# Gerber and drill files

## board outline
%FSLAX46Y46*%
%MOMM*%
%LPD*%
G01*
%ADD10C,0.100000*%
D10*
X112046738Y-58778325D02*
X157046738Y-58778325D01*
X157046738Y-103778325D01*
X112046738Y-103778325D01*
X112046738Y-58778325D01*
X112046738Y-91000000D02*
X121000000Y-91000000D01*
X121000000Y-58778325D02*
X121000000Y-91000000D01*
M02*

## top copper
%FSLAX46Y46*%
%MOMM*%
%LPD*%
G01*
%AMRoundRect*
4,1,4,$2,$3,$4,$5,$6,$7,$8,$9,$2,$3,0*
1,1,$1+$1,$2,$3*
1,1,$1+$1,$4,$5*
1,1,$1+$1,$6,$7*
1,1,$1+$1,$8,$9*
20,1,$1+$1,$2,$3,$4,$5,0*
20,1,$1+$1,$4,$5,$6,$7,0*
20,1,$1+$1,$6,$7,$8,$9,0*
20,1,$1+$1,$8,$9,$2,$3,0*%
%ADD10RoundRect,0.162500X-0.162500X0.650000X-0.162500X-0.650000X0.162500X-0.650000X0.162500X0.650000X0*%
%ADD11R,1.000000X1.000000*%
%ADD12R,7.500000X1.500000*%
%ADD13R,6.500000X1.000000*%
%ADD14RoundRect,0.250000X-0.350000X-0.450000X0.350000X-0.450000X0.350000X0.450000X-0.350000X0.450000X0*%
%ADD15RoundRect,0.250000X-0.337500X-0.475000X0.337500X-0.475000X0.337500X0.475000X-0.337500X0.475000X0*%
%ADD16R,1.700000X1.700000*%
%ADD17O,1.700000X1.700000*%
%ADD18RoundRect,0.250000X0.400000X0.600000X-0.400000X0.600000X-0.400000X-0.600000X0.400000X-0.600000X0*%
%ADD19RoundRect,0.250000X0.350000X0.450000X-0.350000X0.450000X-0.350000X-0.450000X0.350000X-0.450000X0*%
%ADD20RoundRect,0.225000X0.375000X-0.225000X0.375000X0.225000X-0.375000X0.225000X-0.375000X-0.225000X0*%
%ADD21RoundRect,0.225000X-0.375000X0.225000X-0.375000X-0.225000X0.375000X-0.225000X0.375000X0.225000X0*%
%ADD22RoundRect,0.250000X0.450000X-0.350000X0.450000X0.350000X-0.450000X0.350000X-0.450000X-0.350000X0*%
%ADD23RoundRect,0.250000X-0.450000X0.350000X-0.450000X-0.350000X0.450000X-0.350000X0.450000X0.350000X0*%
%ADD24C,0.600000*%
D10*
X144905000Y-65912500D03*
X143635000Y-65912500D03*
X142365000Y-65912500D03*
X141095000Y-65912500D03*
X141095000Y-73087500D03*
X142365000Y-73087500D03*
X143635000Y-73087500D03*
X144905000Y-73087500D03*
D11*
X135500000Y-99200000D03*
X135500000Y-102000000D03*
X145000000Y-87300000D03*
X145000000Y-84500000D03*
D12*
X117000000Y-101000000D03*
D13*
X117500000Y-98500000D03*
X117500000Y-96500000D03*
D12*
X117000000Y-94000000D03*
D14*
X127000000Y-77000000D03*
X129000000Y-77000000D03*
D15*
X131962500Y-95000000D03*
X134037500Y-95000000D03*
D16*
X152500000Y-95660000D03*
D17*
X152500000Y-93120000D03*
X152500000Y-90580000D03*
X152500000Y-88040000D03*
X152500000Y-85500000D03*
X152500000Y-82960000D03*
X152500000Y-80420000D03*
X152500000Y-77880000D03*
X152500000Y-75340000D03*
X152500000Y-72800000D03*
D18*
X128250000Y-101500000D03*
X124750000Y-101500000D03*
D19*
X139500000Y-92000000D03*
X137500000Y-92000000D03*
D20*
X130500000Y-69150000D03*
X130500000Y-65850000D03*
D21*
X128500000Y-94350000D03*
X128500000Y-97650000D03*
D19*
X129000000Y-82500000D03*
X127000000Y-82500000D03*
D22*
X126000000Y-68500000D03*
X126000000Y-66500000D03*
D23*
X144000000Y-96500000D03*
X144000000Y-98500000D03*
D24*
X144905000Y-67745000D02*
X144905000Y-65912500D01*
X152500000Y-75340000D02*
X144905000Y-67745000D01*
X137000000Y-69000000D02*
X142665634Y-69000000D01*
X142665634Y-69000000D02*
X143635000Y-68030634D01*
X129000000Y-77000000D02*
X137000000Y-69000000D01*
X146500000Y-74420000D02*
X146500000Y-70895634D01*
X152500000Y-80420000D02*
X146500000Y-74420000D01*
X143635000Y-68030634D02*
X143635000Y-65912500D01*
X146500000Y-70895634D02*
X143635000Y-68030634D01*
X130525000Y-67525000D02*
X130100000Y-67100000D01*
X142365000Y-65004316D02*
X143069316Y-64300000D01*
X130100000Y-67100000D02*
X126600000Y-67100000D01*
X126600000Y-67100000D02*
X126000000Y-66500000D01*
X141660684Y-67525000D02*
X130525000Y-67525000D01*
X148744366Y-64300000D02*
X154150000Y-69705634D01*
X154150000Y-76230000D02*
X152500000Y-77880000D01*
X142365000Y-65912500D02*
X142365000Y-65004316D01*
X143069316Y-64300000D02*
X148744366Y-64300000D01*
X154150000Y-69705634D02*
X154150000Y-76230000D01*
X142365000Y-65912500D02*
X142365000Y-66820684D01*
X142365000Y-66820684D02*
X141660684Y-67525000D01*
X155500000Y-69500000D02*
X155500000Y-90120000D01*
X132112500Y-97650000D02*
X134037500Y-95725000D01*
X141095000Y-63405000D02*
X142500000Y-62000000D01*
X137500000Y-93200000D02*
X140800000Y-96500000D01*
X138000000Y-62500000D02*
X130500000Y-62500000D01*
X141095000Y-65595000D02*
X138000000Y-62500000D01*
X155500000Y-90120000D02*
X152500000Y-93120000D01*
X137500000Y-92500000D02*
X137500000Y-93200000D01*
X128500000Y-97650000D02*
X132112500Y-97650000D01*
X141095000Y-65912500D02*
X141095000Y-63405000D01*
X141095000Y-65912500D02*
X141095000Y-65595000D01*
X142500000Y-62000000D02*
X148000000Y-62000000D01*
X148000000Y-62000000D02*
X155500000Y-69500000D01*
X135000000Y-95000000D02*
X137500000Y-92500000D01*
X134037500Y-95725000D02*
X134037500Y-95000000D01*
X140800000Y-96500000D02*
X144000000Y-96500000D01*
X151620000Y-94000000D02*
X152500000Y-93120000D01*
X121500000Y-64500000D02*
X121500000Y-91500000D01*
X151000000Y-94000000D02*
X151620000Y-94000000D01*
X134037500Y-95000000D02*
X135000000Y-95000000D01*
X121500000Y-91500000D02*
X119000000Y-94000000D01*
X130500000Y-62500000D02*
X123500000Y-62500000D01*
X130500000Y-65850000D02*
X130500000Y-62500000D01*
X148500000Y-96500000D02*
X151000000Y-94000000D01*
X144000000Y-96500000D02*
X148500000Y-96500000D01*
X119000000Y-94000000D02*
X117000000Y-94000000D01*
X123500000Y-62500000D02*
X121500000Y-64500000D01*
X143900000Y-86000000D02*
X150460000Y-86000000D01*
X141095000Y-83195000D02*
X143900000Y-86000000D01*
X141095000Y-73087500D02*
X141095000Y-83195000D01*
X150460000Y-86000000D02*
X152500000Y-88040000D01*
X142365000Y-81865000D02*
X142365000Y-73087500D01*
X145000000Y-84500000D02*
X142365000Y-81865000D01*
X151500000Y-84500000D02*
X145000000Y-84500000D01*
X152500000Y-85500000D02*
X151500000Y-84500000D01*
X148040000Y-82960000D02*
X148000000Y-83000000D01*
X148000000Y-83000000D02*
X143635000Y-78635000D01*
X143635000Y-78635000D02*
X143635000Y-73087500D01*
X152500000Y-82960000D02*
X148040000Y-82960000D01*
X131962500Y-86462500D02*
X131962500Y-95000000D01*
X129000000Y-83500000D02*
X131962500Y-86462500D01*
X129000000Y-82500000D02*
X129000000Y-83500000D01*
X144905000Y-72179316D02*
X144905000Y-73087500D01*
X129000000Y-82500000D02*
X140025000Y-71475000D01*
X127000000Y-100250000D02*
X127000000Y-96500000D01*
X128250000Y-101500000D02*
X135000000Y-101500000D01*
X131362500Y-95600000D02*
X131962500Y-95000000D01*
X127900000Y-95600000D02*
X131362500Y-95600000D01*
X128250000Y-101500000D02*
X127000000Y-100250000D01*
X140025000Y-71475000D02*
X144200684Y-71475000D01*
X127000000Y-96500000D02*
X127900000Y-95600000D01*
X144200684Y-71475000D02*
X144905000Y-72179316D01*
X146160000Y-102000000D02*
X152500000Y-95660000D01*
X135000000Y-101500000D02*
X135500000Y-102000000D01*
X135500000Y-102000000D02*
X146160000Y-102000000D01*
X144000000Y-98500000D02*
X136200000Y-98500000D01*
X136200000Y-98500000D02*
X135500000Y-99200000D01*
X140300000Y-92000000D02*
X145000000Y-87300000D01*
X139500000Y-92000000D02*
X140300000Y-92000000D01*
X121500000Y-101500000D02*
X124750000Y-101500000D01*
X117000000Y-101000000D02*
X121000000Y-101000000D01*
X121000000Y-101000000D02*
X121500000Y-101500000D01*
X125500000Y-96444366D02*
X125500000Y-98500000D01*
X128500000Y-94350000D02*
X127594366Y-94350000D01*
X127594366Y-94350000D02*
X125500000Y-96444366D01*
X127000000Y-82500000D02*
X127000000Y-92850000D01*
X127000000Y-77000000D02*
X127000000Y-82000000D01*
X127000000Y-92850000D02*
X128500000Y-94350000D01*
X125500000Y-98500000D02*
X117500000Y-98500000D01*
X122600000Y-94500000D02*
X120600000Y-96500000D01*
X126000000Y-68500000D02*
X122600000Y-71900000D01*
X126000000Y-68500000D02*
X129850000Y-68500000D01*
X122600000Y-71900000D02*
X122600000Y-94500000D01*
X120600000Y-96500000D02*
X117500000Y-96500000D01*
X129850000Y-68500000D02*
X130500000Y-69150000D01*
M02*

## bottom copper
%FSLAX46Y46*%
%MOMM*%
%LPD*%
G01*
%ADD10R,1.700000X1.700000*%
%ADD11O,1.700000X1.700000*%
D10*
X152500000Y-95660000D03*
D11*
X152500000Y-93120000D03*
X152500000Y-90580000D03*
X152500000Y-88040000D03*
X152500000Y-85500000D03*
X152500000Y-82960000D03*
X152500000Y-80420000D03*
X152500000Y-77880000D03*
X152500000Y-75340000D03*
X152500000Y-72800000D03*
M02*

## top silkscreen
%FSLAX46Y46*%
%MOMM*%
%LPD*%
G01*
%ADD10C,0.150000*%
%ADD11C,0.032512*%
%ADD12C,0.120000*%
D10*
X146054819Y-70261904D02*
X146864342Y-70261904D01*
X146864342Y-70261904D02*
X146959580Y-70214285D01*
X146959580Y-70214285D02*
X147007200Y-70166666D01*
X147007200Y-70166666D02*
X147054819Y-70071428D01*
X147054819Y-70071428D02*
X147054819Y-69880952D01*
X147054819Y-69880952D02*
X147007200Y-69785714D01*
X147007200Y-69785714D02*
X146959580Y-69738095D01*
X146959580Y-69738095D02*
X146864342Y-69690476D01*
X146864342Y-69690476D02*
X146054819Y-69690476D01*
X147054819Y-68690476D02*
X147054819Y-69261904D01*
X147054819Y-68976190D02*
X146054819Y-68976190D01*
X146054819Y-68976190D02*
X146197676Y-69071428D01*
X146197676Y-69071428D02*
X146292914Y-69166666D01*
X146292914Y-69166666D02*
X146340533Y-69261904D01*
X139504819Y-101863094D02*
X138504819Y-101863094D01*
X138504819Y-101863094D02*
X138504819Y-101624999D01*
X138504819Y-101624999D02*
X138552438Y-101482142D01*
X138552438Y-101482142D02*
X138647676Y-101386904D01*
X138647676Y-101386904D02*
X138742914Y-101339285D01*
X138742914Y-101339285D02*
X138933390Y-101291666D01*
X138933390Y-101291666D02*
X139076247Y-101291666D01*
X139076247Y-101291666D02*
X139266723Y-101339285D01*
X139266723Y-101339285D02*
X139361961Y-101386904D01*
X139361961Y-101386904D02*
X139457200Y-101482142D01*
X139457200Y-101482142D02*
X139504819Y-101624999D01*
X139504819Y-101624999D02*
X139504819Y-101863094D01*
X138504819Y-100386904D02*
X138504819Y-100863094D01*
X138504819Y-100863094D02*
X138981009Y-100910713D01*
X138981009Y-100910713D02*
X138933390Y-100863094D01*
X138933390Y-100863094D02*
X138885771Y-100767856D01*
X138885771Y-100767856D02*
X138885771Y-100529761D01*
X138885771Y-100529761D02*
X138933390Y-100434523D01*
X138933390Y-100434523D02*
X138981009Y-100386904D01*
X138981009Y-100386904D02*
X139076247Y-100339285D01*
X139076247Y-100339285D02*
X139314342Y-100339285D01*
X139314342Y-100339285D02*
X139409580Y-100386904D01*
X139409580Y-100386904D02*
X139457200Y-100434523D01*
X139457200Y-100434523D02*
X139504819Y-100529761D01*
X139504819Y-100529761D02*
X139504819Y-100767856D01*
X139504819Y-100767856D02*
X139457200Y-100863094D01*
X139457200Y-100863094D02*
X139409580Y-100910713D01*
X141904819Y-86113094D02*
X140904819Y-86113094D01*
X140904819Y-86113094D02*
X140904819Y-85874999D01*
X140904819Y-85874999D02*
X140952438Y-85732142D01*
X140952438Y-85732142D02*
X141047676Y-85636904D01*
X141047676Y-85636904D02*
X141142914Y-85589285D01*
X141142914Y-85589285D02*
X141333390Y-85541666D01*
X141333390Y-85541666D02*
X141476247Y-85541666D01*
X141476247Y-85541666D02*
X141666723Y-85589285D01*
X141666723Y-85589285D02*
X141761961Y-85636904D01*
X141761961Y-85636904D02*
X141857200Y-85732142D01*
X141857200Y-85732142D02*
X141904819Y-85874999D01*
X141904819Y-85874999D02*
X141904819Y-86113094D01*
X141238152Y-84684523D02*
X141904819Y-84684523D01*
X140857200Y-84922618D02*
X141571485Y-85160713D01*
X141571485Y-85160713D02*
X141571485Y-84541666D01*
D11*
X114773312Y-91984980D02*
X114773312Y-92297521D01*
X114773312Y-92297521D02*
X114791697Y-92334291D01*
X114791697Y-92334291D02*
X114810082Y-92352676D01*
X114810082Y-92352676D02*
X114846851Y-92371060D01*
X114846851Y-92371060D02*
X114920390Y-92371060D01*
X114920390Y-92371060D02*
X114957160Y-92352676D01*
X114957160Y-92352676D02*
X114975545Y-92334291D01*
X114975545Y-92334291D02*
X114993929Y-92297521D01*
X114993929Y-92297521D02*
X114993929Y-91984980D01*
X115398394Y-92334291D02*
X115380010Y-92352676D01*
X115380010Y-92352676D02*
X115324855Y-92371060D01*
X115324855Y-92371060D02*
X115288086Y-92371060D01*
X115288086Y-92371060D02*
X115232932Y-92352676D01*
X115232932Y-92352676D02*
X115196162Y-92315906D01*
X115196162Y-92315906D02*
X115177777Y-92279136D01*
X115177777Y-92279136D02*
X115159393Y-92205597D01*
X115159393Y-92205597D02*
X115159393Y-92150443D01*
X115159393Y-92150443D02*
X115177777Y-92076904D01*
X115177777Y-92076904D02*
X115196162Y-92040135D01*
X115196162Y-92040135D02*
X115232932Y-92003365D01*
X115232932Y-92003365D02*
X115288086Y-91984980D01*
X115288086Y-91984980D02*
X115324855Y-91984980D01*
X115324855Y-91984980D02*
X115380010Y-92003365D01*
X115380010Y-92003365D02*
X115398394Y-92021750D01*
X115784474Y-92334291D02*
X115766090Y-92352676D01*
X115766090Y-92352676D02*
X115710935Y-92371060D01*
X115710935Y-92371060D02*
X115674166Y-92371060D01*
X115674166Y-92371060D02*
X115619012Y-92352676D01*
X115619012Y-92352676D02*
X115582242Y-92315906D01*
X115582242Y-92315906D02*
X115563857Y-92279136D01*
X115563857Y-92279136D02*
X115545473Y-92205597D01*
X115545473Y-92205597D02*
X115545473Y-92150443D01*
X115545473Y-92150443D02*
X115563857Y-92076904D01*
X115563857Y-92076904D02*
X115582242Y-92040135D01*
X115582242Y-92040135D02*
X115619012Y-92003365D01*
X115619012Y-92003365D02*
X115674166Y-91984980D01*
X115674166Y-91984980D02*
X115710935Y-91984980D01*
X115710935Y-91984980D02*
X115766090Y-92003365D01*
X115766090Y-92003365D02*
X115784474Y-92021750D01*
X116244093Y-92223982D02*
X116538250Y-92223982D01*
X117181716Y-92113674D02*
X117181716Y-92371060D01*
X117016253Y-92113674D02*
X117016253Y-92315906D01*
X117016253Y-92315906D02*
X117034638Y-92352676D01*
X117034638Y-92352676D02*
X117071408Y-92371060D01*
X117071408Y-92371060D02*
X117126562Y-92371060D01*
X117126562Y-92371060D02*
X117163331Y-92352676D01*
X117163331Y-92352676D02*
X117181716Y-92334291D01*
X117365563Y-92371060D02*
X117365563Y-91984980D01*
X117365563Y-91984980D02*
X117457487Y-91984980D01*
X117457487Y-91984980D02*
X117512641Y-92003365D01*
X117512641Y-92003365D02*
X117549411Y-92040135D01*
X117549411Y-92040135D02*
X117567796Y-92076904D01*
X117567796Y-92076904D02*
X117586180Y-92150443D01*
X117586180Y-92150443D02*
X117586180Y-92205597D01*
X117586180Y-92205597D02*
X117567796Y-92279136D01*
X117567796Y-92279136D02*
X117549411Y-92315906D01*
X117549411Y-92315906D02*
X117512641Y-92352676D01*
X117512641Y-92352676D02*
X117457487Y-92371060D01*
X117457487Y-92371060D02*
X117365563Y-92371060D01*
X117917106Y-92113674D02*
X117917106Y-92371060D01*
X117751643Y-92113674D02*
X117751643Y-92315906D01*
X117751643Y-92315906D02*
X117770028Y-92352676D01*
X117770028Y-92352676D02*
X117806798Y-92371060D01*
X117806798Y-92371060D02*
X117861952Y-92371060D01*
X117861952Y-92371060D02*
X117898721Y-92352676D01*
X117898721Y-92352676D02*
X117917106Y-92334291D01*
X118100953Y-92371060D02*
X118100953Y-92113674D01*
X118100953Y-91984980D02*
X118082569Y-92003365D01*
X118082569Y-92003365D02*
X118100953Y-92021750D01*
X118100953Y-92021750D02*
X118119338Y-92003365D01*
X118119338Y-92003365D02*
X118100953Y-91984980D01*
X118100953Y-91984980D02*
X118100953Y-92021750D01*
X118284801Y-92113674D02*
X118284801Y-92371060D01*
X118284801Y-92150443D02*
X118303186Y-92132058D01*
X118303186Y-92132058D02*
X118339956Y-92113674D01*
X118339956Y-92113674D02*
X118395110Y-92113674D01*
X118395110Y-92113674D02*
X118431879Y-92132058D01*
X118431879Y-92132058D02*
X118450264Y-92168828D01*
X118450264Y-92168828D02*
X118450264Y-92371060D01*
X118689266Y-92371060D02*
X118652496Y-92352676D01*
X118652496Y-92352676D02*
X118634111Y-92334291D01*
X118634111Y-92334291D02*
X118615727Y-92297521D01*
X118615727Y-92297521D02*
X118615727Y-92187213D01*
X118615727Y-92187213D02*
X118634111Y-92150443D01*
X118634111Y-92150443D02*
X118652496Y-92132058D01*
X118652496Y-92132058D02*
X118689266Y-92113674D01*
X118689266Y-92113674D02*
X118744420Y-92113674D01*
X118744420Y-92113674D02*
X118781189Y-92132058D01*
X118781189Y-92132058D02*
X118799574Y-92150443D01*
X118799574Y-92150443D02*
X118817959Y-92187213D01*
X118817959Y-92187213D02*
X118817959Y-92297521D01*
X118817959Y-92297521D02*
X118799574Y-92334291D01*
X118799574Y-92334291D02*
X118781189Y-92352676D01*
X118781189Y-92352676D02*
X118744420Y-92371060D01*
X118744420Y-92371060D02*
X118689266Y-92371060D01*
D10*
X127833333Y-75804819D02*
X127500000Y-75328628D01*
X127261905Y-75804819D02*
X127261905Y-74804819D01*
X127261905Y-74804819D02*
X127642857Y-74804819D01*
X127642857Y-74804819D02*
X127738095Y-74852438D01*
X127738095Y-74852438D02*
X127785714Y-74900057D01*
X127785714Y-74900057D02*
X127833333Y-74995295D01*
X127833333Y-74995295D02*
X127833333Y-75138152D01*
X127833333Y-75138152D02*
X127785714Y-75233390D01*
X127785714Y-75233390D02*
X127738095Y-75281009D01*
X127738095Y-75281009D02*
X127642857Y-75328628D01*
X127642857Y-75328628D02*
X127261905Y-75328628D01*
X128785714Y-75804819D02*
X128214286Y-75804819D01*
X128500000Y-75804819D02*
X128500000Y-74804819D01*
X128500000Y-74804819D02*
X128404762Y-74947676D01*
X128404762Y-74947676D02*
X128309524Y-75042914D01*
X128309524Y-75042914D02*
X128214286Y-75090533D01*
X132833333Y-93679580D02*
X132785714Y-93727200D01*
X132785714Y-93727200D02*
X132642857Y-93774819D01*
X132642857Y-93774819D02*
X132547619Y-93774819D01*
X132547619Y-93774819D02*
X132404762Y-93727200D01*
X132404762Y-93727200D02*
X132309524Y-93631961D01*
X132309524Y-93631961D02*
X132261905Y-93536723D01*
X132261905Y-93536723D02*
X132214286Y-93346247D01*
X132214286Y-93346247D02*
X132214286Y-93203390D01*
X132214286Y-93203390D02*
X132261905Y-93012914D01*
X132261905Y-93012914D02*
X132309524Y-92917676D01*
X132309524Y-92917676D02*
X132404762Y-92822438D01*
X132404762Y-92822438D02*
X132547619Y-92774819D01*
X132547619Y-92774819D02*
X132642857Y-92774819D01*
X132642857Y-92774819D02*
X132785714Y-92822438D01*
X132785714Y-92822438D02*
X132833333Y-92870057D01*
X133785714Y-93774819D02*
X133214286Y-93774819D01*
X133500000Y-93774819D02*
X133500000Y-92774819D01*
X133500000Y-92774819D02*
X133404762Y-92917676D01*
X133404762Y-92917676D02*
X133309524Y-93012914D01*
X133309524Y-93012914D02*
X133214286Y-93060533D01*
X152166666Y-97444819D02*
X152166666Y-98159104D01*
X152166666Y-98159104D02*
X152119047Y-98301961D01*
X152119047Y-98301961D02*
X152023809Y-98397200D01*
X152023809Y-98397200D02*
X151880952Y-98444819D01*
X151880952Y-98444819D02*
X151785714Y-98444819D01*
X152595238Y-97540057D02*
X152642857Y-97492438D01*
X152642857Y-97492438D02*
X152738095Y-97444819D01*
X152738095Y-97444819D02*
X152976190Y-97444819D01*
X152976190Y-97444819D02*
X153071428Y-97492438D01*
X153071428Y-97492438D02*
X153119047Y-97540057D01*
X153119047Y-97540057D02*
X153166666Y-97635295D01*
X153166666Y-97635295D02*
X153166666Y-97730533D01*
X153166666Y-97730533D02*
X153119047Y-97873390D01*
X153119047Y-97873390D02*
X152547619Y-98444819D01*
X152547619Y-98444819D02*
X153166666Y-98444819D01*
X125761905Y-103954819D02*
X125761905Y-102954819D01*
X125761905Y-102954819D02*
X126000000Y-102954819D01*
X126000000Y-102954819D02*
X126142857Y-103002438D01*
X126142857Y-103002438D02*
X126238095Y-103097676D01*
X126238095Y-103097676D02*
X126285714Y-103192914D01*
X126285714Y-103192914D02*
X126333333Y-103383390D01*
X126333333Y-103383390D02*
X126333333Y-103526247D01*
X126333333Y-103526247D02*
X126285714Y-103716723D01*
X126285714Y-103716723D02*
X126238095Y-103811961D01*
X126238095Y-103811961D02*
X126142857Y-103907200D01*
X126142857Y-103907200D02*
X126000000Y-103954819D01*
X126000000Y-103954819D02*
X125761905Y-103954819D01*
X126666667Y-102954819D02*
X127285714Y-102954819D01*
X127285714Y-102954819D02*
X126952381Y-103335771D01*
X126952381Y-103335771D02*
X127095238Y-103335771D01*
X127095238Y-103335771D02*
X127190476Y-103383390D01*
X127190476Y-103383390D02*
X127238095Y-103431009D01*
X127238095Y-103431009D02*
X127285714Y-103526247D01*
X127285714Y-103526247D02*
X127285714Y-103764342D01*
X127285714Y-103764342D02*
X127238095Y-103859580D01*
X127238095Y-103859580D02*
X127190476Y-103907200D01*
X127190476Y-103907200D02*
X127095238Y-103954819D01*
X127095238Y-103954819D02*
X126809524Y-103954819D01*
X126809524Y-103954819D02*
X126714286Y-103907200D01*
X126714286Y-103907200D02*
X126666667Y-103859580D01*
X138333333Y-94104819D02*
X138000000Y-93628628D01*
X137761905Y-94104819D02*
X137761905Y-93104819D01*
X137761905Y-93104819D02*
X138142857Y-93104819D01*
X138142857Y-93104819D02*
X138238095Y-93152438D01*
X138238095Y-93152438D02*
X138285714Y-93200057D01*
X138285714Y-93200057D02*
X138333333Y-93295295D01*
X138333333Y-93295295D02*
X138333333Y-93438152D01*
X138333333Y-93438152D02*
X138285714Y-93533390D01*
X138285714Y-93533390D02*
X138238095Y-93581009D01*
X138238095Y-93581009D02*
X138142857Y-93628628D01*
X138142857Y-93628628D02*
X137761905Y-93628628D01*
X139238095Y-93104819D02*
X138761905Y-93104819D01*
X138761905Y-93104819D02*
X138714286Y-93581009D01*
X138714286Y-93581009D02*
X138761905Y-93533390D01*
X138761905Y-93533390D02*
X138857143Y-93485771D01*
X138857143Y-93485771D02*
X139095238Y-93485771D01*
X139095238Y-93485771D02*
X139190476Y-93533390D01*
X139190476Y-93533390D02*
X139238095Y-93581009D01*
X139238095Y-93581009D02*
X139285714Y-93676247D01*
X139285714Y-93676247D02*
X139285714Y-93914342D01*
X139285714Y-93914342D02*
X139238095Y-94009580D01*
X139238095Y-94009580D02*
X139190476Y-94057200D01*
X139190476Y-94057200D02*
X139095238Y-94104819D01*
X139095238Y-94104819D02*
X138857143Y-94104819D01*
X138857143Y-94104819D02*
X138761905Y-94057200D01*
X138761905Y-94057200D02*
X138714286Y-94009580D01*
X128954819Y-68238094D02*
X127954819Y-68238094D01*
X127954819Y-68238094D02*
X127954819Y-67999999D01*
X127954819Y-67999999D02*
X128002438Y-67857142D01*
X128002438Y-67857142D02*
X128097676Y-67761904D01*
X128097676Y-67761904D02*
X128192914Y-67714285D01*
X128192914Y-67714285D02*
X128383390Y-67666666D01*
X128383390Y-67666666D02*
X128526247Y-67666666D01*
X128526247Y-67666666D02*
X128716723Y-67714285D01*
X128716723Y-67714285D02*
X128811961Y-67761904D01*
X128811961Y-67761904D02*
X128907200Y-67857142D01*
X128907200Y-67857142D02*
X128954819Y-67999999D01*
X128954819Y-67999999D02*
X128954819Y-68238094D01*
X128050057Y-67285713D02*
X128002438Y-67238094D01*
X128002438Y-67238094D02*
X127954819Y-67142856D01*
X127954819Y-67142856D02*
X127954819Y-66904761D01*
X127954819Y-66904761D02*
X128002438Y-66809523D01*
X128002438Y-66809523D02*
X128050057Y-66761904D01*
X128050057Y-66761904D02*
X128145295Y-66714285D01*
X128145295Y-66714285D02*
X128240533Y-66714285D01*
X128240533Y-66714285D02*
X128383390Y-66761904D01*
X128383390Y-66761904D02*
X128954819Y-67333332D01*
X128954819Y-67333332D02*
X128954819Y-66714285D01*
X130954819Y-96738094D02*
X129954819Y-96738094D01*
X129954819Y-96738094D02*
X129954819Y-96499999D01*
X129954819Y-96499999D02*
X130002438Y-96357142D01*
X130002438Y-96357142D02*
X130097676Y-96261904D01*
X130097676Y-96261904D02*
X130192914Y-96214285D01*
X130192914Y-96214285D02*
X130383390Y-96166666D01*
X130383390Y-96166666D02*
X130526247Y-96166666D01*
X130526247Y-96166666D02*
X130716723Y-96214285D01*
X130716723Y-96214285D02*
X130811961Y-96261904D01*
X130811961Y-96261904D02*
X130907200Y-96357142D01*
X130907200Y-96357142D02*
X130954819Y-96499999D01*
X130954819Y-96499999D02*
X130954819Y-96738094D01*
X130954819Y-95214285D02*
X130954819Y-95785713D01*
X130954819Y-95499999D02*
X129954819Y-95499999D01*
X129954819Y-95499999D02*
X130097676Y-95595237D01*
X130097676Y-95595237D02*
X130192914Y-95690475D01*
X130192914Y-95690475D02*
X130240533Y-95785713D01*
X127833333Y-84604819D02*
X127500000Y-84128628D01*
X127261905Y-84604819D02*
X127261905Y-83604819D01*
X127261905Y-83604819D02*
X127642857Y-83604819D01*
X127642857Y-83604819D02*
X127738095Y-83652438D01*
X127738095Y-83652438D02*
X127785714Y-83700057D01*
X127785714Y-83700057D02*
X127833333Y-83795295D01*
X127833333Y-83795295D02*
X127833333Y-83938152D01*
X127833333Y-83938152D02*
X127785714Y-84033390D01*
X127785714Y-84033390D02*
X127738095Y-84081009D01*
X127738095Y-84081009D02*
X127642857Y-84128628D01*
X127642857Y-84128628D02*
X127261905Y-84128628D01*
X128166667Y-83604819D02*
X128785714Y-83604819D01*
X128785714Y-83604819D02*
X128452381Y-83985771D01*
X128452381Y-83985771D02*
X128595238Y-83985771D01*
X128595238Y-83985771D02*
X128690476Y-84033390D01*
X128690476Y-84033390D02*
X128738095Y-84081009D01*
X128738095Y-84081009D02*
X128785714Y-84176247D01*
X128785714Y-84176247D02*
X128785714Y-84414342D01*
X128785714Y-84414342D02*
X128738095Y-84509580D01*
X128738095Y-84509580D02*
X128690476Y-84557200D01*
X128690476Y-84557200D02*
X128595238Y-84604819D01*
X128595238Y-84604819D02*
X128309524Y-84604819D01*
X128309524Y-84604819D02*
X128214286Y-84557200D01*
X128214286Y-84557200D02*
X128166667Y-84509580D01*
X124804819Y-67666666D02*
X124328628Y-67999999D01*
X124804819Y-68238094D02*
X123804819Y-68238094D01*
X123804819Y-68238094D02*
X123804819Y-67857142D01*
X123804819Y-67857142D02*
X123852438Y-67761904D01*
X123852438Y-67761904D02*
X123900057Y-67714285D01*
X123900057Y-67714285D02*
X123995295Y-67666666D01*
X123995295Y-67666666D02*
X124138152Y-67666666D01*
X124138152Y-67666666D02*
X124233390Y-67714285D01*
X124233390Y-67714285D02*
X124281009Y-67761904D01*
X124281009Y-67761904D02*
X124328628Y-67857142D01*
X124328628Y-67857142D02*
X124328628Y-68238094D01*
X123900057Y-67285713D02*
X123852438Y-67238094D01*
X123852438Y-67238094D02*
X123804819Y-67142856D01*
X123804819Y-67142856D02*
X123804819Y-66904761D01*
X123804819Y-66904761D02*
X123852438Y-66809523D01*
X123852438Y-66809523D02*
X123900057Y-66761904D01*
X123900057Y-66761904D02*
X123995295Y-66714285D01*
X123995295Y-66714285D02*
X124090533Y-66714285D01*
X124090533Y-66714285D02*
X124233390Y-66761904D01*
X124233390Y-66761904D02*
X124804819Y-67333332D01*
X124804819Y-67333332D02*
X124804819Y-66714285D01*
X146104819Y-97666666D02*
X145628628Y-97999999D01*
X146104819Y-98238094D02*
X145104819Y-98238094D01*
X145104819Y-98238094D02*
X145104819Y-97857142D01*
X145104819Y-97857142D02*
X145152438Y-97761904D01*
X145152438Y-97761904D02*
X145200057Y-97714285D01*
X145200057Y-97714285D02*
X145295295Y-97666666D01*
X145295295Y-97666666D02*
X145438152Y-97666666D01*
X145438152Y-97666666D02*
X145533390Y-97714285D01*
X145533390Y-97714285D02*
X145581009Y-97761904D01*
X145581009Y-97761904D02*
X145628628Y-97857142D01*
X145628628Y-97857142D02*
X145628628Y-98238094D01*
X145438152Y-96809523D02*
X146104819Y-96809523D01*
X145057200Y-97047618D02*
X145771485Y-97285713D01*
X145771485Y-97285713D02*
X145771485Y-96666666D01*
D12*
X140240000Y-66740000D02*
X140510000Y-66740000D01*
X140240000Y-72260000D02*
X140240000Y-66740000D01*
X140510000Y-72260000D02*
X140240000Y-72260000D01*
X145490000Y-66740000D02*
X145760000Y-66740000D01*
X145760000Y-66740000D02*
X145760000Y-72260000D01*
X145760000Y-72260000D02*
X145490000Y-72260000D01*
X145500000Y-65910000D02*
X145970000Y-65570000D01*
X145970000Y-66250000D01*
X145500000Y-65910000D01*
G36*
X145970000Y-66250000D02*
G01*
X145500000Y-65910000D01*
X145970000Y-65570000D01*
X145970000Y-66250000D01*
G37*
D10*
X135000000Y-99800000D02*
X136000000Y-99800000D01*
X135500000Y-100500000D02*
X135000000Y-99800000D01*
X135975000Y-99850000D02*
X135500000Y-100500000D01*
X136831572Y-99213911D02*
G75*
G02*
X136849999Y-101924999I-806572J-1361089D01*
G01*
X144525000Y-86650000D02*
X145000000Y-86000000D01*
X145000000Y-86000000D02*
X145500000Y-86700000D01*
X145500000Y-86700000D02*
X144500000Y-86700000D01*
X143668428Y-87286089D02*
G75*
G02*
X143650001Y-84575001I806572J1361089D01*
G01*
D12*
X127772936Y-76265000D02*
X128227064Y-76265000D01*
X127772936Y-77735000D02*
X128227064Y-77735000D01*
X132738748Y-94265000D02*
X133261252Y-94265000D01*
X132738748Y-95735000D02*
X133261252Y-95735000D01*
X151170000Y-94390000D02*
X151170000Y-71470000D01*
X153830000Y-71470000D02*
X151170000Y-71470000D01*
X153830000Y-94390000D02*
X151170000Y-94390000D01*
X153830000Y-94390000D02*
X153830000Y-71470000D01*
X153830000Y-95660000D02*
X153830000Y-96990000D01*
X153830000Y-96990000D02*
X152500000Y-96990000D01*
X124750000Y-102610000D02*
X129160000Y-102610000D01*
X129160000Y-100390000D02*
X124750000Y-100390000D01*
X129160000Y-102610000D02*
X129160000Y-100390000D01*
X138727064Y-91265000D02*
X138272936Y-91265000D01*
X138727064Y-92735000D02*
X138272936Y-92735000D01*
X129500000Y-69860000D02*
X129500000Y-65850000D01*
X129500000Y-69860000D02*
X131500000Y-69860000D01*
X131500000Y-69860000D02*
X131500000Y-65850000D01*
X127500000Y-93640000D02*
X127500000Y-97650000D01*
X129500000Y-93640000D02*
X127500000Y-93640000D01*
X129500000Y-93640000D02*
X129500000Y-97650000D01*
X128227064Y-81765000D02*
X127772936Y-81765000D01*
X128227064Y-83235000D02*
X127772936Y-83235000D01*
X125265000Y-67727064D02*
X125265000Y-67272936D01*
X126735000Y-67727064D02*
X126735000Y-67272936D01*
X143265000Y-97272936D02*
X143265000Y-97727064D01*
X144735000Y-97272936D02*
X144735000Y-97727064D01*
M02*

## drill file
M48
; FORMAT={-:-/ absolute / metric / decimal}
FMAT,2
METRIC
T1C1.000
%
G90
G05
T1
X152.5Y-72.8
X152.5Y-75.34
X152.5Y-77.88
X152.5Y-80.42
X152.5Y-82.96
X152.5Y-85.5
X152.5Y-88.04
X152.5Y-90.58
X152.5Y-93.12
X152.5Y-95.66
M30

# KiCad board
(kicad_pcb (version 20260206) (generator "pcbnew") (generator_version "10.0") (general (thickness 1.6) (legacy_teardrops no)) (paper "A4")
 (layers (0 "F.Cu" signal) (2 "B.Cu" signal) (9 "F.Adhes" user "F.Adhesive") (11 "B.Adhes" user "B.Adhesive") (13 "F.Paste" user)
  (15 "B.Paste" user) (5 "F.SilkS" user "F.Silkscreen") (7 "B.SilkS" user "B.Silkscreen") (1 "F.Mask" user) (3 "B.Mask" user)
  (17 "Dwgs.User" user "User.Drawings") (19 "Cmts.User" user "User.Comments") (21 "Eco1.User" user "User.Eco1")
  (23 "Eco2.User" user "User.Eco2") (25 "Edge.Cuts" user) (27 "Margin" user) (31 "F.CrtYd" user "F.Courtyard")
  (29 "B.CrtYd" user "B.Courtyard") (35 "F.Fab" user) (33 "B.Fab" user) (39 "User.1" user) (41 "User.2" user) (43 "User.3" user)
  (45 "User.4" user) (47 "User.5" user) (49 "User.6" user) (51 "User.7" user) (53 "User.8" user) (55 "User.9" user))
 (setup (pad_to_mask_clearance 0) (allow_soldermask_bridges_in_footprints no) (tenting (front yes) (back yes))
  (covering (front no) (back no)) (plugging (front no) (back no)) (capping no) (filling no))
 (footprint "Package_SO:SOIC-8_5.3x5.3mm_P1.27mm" (layer "F.Cu") (at 143 69.5 -90)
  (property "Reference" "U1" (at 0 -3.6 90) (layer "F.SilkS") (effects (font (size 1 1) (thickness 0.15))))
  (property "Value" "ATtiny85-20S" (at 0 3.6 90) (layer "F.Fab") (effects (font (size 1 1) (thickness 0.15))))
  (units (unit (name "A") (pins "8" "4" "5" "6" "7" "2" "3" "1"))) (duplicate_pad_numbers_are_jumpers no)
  (fp_line (start -2.76 2.76) (end -2.76 2.49) (stroke (width 0.12) (type solid)) (layer "F.SilkS"))
  (fp_line (start 2.76 2.76) (end -2.76 2.76) (stroke (width 0.12) (type solid)) (layer "F.SilkS"))
  (fp_line (start 2.76 2.49) (end 2.76 2.76) (stroke (width 0.12) (type solid)) (layer "F.SilkS"))
  (fp_line (start -2.76 -2.49) (end -2.76 -2.76) (stroke (width 0.12) (type solid)) (layer "F.SilkS"))
  (fp_line (start -2.76 -2.76) (end 2.76 -2.76) (stroke (width 0.12) (type solid)) (layer "F.SilkS"))
  (fp_line (start 2.76 -2.76) (end 2.76 -2.49) (stroke (width 0.12) (type solid)) (layer "F.SilkS"))
  (fp_poly (pts (xy -3.59 -2.5) (xy -3.93 -2.97) (xy -3.25 -2.97)) (stroke (width 0.12) (type solid)) (fill yes) (layer "F.SilkS"))
  (pad "1" smd roundrect (at -3.5875 -1.905 270) (size 1.625 0.65) (layers "F.Cu" "F.Mask" "F.Paste") (roundrect_rratio 0.25)
   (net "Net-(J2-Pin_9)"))
  (pad "2" smd roundrect (at -3.5875 -0.635 270) (size 1.625 0.65) (layers "F.Cu" "F.Mask" "F.Paste") (roundrect_rratio 0.25)
   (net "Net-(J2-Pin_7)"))
  (pad "3" smd roundrect (at -3.5875 0.635 270) (size 1.625 0.65) (layers "F.Cu" "F.Mask" "F.Paste") (roundrect_rratio 0.25)
   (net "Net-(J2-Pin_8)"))
  (pad "4" smd roundrect (at -3.5875 1.905 270) (size 1.625 0.65) (layers "F.Cu" "F.Mask" "F.Paste") (roundrect_rratio 0.25) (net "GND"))
  (pad "5" smd roundrect (at 3.5875 1.905 270) (size 1.625 0.65) (layers "F.Cu" "F.Mask" "F.Paste") (roundrect_rratio 0.25)
   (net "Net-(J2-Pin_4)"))
  (pad "6" smd roundrect (at 3.5875 0.635 270) (size 1.625 0.65) (layers "F.Cu" "F.Mask" "F.Paste") (roundrect_rratio 0.25)
   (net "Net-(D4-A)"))
  (pad "7" smd roundrect (at 3.5875 -0.635 270) (size 1.625 0.65) (layers "F.Cu" "F.Mask" "F.Paste") (roundrect_rratio 0.25)
   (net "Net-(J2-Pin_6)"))
  (pad "8" smd roundrect (at 3.5875 -1.905 270) (size 1.625 0.65) (layers "F.Cu" "F.Mask" "F.Paste") (roundrect_rratio 0.25) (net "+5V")))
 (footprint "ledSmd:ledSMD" (layer "F.Cu") (at 135.5 101 -90)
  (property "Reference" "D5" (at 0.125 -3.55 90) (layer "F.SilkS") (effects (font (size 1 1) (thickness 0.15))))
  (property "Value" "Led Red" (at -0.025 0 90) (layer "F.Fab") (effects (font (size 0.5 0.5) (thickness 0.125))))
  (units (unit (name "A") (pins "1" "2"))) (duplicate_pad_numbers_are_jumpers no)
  (fp_line (start -1.2 0.5) (end -1.2 -0.5) (stroke (width 0.15) (type solid)) (layer "F.SilkS"))
  (fp_line (start -0.5 0) (end -1.2 0.5) (stroke (width 0.15) (type solid)) (layer "F.SilkS"))
  (fp_line (start -1.15 -0.475) (end -0.5 0) (stroke (width 0.15) (type solid)) (layer "F.SilkS"))
  (fp_arc (start -1.786089 -1.331572) (mid -0.435753 -2.107089) (end 0.924999 -1.349999) (stroke (width 0.15) (type solid))
   (layer "F.SilkS"))
  (pad "1" smd rect (at -1.8 0 270) (size 1 1) (layers "F.Cu" "F.Mask" "F.Paste") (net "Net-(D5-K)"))
  (pad "2" smd rect (at 1 0 270) (size 1 1) (layers "F.Cu" "F.Mask" "F.Paste") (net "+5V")))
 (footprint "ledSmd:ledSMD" (layer "F.Cu") (at 145 85.5 90)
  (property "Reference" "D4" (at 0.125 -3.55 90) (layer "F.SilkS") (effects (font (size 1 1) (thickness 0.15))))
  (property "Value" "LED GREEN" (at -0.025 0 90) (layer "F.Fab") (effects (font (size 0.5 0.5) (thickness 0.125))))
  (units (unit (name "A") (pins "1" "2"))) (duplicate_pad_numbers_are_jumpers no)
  (fp_line (start -1.15 -0.475) (end -0.5 0) (stroke (width 0.15) (type solid)) (layer "F.SilkS"))
  (fp_line (start -0.5 0) (end -1.2 0.5) (stroke (width 0.15) (type solid)) (layer "F.SilkS"))
  (fp_line (start -1.2 0.5) (end -1.2 -0.5) (stroke (width 0.15) (type solid)) (layer "F.SilkS"))
  (fp_arc (start -1.786089 -1.331572) (mid -0.435753 -2.107089) (end 0.924999 -1.349999) (stroke (width 0.15) (type solid))
   (layer "F.SilkS"))
  (pad "1" smd rect (at -1.8 0 90) (size 1 1) (layers "F.Cu" "F.Mask" "F.Paste") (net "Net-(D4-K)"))
  (pad "2" smd rect (at 1 0 90) (size 1 1) (layers "F.Cu" "F.Mask" "F.Paste") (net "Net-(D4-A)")))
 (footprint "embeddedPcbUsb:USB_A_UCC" (layer "F.Cu") (at 117.2 97.5)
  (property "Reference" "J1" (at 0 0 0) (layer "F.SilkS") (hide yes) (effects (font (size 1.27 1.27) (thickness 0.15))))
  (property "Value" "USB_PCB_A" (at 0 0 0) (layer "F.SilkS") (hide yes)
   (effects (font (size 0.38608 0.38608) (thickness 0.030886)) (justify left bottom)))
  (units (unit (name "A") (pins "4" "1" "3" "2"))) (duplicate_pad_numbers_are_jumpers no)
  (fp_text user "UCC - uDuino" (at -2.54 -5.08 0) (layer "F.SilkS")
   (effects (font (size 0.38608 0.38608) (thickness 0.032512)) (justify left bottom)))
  (pad "1" smd rect (at -0.2 3.5) (size 7.5 1.5) (layers "F.Cu" "F.Mask" "F.Paste") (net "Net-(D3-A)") (solder_mask_margin 0.1016))
  (pad "2" smd rect (at 0.3 1) (size 6.5 1) (layers "F.Cu" "F.Mask" "F.Paste") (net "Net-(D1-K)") (solder_mask_margin 0.1016))
  (pad "3" smd rect (at 0.3 -1) (size 6.5 1) (layers "F.Cu" "F.Mask" "F.Paste") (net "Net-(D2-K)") (solder_mask_margin 0.1016))
  (pad "4" smd rect (at -0.2 -3.5) (size 7.5 1.5) (layers "F.Cu" "F.Mask" "F.Paste") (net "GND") (solder_mask_margin 0.1016)))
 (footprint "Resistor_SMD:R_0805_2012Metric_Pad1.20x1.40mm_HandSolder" (layer "F.Cu") (at 128 77)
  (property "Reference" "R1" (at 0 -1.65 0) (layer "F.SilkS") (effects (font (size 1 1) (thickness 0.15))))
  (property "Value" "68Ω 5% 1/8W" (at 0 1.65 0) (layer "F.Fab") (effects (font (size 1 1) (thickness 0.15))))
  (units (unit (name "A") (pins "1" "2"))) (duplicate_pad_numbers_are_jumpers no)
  (fp_line (start -0.227064 -0.735) (end 0.227064 -0.735) (stroke (width 0.12) (type solid)) (layer "F.SilkS"))
  (fp_line (start -0.227064 0.735) (end 0.227064 0.735) (stroke (width 0.12) (type solid)) (layer "F.SilkS"))
  (pad "1" smd roundrect (at -1 0) (size 1.2 1.4) (layers "F.Cu" "F.Mask" "F.Paste") (roundrect_rratio 0.208333) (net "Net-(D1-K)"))
  (pad "2" smd roundrect (at 1 0) (size 1.2 1.4) (layers "F.Cu" "F.Mask" "F.Paste") (roundrect_rratio 0.208333) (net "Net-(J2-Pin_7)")))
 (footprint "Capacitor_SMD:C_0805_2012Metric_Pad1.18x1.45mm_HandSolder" (layer "F.Cu") (at 133 95)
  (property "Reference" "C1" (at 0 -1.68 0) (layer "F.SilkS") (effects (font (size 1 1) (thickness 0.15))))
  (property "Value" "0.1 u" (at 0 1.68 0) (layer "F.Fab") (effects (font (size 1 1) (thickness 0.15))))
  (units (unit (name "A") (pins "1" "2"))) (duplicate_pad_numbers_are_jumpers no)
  (fp_line (start -0.261252 -0.735) (end 0.261252 -0.735) (stroke (width 0.12) (type solid)) (layer "F.SilkS"))
  (fp_line (start -0.261252 0.735) (end 0.261252 0.735) (stroke (width 0.12) (type solid)) (layer "F.SilkS"))
  (pad "1" smd roundrect (at -1.0375 0) (size 1.175 1.45) (layers "F.Cu" "F.Mask" "F.Paste") (roundrect_rratio 0.212766) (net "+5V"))
  (pad "2" smd roundrect (at 1.0375 0) (size 1.175 1.45) (layers "F.Cu" "F.Mask" "F.Paste") (roundrect_rratio 0.212766) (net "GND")))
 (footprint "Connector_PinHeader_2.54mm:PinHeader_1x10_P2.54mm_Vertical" (layer "F.Cu") (at 152.5 95.66 180)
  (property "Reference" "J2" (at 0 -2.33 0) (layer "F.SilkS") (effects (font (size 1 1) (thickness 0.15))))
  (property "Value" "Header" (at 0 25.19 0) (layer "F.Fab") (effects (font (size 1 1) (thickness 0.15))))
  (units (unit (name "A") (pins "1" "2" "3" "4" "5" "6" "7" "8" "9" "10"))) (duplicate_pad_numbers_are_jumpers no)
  (fp_line (start 1.33 1.27) (end 1.33 24.19) (stroke (width 0.12) (type solid)) (layer "F.SilkS"))
  (fp_line (start -1.33 24.19) (end 1.33 24.19) (stroke (width 0.12) (type solid)) (layer "F.SilkS"))
  (fp_line (start -1.33 1.27) (end 1.33 1.27) (stroke (width 0.12) (type solid)) (layer "F.SilkS"))
  (fp_line (start -1.33 1.27) (end -1.33 24.19) (stroke (width 0.12) (type solid)) (layer "F.SilkS"))
  (fp_line (start -1.33 0) (end -1.33 -1.33) (stroke (width 0.12) (type solid)) (layer "F.SilkS"))
  (fp_line (start -1.33 -1.33) (end 0 -1.33) (stroke (width 0.12) (type solid)) (layer "F.SilkS"))
  (pad "1" thru_hole rect (at 0 0 180) (size 1.7 1.7) (drill 1) (layers "*.Cu" "*.Mask") (remove_unused_layers no) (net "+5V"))
  (pad "2" thru_hole oval (at 0 2.54 180) (size 1.7 1.7) (drill 1) (layers "*.Cu" "*.Mask") (remove_unused_layers no) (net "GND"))
  (pad "3" thru_hole oval (at 0 5.08 180) (size 1.7 1.7) (drill 1) (layers "*.Cu" "*.Mask") (remove_unused_layers no)
   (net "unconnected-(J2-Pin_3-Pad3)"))
  (pad "4" thru_hole oval (at 0 7.62 180) (size 1.7 1.7) (drill 1) (layers "*.Cu" "*.Mask") (remove_unused_layers no) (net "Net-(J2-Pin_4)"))
  (pad "5" thru_hole oval (at 0 10.16 180) (size 1.7 1.7) (drill 1) (layers "*.Cu" "*.Mask") (remove_unused_layers no) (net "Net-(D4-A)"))
  (pad "6" thru_hole oval (at 0 12.7 180) (size 1.7 1.7) (drill 1) (layers "*.Cu" "*.Mask") (remove_unused_layers no) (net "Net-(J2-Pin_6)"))
  (pad "7" thru_hole oval (at 0 15.24 180) (size 1.7 1.7) (drill 1) (layers "*.Cu" "*.Mask") (remove_unused_layers no)
   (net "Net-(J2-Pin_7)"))
  (pad "8" thru_hole oval (at 0 17.78 180) (size 1.7 1.7) (drill 1) (layers "*.Cu" "*.Mask") (remove_unused_layers no)
   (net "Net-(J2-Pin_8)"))
  (pad "9" thru_hole oval (at 0 20.32 180) (size 1.7 1.7) (drill 1) (layers "*.Cu" "*.Mask") (remove_unused_layers no)
   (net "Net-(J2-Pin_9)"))
  (pad "10" thru_hole oval (at 0 22.86 180) (size 1.7 1.7) (drill 1) (layers "*.Cu" "*.Mask") (remove_unused_layers no)
   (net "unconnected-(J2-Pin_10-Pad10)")))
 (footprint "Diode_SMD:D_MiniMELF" (layer "F.Cu") (at 126.5 101.5 180)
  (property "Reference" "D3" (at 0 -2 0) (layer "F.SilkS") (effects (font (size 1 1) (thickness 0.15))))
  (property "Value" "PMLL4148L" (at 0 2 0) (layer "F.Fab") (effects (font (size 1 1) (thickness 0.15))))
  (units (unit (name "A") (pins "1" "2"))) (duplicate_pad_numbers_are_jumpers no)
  (fp_line (start 1.75 -1.11) (end -2.66 -1.11) (stroke (width 0.12) (type solid)) (layer "F.SilkS"))
  (fp_line (start -2.66 1.11) (end 1.75 1.11) (stroke (width 0.12) (type solid)) (layer "F.SilkS"))
  (fp_line (start -2.66 -1.11) (end -2.66 1.11) (stroke (width 0.12) (type solid)) (layer "F.SilkS"))
  (pad "1" smd roundrect (at -1.75 0 180) (size 1.3 1.7) (layers "F.Cu" "F.Mask" "F.Paste") (roundrect_rratio 0.1923076923) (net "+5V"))
  (pad "2" smd roundrect (at 1.75 0 180) (size 1.3 1.7) (layers "F.Cu" "F.Mask" "F.Paste") (roundrect_rratio 0.1923076923)
   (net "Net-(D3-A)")))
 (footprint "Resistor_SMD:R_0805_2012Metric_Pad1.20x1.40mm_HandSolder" (layer "F.Cu") (at 138.5 92 180)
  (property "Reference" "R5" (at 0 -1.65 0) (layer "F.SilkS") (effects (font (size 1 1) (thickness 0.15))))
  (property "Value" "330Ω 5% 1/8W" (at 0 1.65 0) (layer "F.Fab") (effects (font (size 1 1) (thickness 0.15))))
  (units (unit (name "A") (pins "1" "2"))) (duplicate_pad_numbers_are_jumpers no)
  (fp_line (start -0.227064 0.735) (end 0.227064 0.735) (stroke (width 0.12) (type solid)) (layer "F.SilkS"))
  (fp_line (start -0.227064 -0.735) (end 0.227064 -0.735) (stroke (width 0.12) (type solid)) (layer "F.SilkS"))
  (pad "1" smd roundrect (at -1 0 180) (size 1.2 1.4) (layers "F.Cu" "F.Mask" "F.Paste") (roundrect_rratio 0.208333) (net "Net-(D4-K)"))
  (pad "2" smd roundrect (at 1 0 180) (size 1.2 1.4) (layers "F.Cu" "F.Mask" "F.Paste") (roundrect_rratio 0.208333) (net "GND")))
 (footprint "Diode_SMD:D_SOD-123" (layer "F.Cu") (at 130.5 67.5 90)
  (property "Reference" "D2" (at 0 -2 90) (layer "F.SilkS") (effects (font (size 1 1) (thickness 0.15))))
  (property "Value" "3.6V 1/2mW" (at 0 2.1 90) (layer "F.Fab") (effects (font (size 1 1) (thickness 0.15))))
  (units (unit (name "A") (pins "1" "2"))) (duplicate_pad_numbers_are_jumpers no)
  (fp_line (start -2.36 -1) (end 1.65 -1) (stroke (width 0.12) (type solid)) (layer "F.SilkS"))
  (fp_line (start -2.36 -1) (end -2.36 1) (stroke (width 0.12) (type solid)) (layer "F.SilkS"))
  (fp_line (start -2.36 1) (end 1.65 1) (stroke (width 0.12) (type solid)) (layer "F.SilkS"))
  (pad "1" smd roundrect (at -1.65 0 90) (size 0.9 1.2) (layers "F.Cu" "F.Mask" "F.Paste") (roundrect_rratio 0.25) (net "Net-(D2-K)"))
  (pad "2" smd roundrect (at 1.65 0 90) (size 0.9 1.2) (layers "F.Cu" "F.Mask" "F.Paste") (roundrect_rratio 0.25) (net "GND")))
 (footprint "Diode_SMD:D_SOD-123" (layer "F.Cu") (at 128.5 96 -90)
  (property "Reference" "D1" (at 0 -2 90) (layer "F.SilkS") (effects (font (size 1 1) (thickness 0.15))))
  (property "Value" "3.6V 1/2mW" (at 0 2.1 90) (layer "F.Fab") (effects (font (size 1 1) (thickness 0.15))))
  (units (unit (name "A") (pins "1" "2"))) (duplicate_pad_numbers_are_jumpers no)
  (fp_line (start -2.36 1) (end 1.65 1) (stroke (width 0.12) (type solid)) (layer "F.SilkS"))
  (fp_line (start -2.36 -1) (end -2.36 1) (stroke (width 0.12) (type solid)) (layer "F.SilkS"))
  (fp_line (start -2.36 -1) (end 1.65 -1) (stroke (width 0.12) (type solid)) (layer "F.SilkS"))
  (pad "1" smd roundrect (at -1.65 0 270) (size 0.9 1.2) (layers "F.Cu" "F.Mask" "F.Paste") (roundrect_rratio 0.25) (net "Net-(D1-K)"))
  (pad "2" smd roundrect (at 1.65 0 270) (size 0.9 1.2) (layers "F.Cu" "F.Mask" "F.Paste") (roundrect_rratio 0.25) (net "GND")))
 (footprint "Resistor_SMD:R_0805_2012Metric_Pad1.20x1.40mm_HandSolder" (layer "F.Cu") (at 128 82.5 180)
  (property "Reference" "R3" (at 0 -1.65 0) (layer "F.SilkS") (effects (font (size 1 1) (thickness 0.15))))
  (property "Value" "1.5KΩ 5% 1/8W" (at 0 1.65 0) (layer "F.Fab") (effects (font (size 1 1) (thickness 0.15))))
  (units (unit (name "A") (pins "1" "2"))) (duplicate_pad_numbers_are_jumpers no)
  (fp_line (start -0.227064 0.735) (end 0.227064 0.735) (stroke (width 0.12) (type solid)) (layer "F.SilkS"))
  (fp_line (start -0.227064 -0.735) (end 0.227064 -0.735) (stroke (width 0.12) (type solid)) (layer "F.SilkS"))
  (pad "1" smd roundrect (at -1 0 180) (size 1.2 1.4) (layers "F.Cu" "F.Mask" "F.Paste") (roundrect_rratio 0.208333) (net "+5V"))
  (pad "2" smd roundrect (at 1 0 180) (size 1.2 1.4) (layers "F.Cu" "F.Mask" "F.Paste") (roundrect_rratio 0.208333) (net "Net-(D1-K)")))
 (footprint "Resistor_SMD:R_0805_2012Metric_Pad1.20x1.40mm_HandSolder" (layer "F.Cu") (at 126 67.5 90)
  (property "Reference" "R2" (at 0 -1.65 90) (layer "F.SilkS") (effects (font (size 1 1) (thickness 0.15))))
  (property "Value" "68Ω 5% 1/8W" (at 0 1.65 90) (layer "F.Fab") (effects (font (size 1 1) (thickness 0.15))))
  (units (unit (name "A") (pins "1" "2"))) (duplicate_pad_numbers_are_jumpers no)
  (fp_line (start -0.227064 -0.735) (end 0.227064 -0.735) (stroke (width 0.12) (type solid)) (layer "F.SilkS"))
  (fp_line (start -0.227064 0.735) (end 0.227064 0.735) (stroke (width 0.12) (type solid)) (layer "F.SilkS"))
  (pad "1" smd roundrect (at -1 0 90) (size 1.2 1.4) (layers "F.Cu" "F.Mask" "F.Paste") (roundrect_rratio 0.208333) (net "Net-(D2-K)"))
  (pad "2" smd roundrect (at 1 0 90) (size 1.2 1.4) (layers "F.Cu" "F.Mask" "F.Paste") (roundrect_rratio 0.208333) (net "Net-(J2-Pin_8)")))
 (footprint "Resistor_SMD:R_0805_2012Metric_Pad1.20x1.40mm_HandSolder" (layer "F.Cu") (at 144 97.5 -90)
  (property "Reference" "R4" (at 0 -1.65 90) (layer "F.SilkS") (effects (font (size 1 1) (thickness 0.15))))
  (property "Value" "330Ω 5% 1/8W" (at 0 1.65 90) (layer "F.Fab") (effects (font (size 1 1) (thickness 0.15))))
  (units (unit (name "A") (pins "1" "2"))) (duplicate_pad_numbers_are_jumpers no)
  (fp_line (start -0.227064 0.735) (end 0.227064 0.735) (stroke (width 0.12) (type solid)) (layer "F.SilkS"))
  (fp_line (start -0.227064 -0.735) (end 0.227064 -0.735) (stroke (width 0.12) (type solid)) (layer "F.SilkS"))
  (pad "1" smd roundrect (at -1 0 270) (size 1.2 1.4) (layers "F.Cu" "F.Mask" "F.Paste") (roundrect_rratio 0.208333) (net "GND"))
  (pad "2" smd roundrect (at 1 0 270) (size 1.2 1.4) (layers "F.Cu" "F.Mask" "F.Paste") (roundrect_rratio 0.208333) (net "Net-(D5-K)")))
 (gr_rect (start 112.046738 58.778325) (end 157.046738 103.778325) (stroke (width 0.1) (type solid)) (fill no) (layer "Edge.Cuts"))
 (gr_line (start 112.046738 91) (end 121 91) (stroke (width 0.1) (type solid)) (layer "Edge.Cuts"))
 (gr_line (start 121 58.778325) (end 121 91) (stroke (width 0.1) (type solid)) (layer "Edge.Cuts"))
 (segment (start 144.905 67.745) (end 144.905 65.9125) (width 0.6) (layer "F.Cu") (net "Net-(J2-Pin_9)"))
 (segment (start 152.5 75.34) (end 144.905 67.745) (width 0.6) (layer "F.Cu") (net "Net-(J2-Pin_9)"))
 (segment (start 137 69) (end 142.665634 69) (width 0.6) (layer "F.Cu") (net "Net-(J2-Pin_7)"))
 (segment (start 142.665634 69) (end 143.635 68.030634) (width 0.6) (layer "F.Cu") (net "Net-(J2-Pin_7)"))
 (segment (start 129 77) (end 137 69) (width 0.6) (layer "F.Cu") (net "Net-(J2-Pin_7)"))
 (segment (start 146.5 74.42) (end 146.5 70.895634) (width 0.6) (layer "F.Cu") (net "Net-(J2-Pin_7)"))
 (segment (start 152.5 80.42) (end 146.5 74.42) (width 0.6) (layer "F.Cu") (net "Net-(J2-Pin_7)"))
 (segment (start 143.635 68.030634) (end 143.635 65.9125) (width 0.6) (layer "F.Cu") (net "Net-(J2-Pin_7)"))
 (segment (start 146.5 70.895634) (end 143.635 68.030634) (width 0.6) (layer "F.Cu") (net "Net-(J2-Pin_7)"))
 (segment (start 130.525 67.525) (end 130.1 67.1) (width 0.6) (layer "F.Cu") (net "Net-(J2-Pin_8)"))
 (segment (start 142.365 65.004316) (end 143.069316 64.3) (width 0.6) (layer "F.Cu") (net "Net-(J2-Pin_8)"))
 (segment (start 130.1 67.1) (end 126.6 67.1) (width 0.6) (layer "F.Cu") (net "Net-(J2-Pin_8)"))
 (segment (start 126.6 67.1) (end 126 66.5) (width 0.6) (layer "F.Cu") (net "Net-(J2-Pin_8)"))
 (segment (start 141.660684 67.525) (end 130.525 67.525) (width 0.6) (layer "F.Cu") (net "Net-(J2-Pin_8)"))
 (segment (start 148.744366 64.3) (end 154.15 69.705634) (width 0.6) (layer "F.Cu") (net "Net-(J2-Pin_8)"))
 (segment (start 154.15 76.23) (end 152.5 77.88) (width 0.6) (layer "F.Cu") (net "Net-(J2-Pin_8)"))
 (segment (start 142.365 65.9125) (end 142.365 65.004316) (width 0.6) (layer "F.Cu") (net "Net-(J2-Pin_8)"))
 (segment (start 143.069316 64.3) (end 148.744366 64.3) (width 0.6) (layer "F.Cu") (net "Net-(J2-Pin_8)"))
 (segment (start 154.15 69.705634) (end 154.15 76.23) (width 0.6) (layer "F.Cu") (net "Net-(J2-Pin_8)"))
 (segment (start 142.365 65.9125) (end 142.365 66.820684) (width 0.6) (layer "F.Cu") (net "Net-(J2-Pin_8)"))
 (segment (start 142.365 66.820684) (end 141.660684 67.525) (width 0.6) (layer "F.Cu") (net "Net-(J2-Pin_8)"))
 (segment (start 155.5 69.5) (end 155.5 90.12) (width 0.6) (layer "F.Cu") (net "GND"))
 (segment (start 132.1125 97.65) (end 134.0375 95.725) (width 0.6) (layer "F.Cu") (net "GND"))
 (segment (start 141.095 63.405) (end 142.5 62) (width 0.6) (layer "F.Cu") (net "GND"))
 (segment (start 137.5 93.2) (end 140.8 96.5) (width 0.6) (layer "F.Cu") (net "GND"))
 (segment (start 138 62.5) (end 130.5 62.5) (width 0.6) (layer "F.Cu") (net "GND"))
 (segment (start 141.095 65.595) (end 138 62.5) (width 0.6) (layer "F.Cu") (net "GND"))
 (segment (start 155.5 90.12) (end 152.5 93.12) (width 0.6) (layer "F.Cu") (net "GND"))
 (segment (start 137.5 92.5) (end 137.5 93.2) (width 0.6) (layer "F.Cu") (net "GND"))
 (segment (start 128.5 97.65) (end 132.1125 97.65) (width 0.6) (layer "F.Cu") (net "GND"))
 (segment (start 141.095 65.9125) (end 141.095 63.405) (width 0.6) (layer "F.Cu") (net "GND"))
 (segment (start 141.095 65.9125) (end 141.095 65.595) (width 0.6) (layer "F.Cu") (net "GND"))
 (segment (start 142.5 62) (end 148 62) (width 0.6) (layer "F.Cu") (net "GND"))
 (segment (start 148 62) (end 155.5 69.5) (width 0.6) (layer "F.Cu") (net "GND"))
 (segment (start 135 95) (end 137.5 92.5) (width 0.6) (layer "F.Cu") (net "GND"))
 (segment (start 134.0375 95.725) (end 134.0375 95) (width 0.6) (layer "F.Cu") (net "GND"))
 (segment (start 140.8 96.5) (end 144 96.5) (width 0.6) (layer "F.Cu") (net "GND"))
 (segment (start 151.62 94) (end 152.5 93.12) (width 0.6) (layer "F.Cu") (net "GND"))
 (segment (start 121.5 64.5) (end 121.5 91.5) (width 0.6) (layer "F.Cu") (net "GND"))
 (segment (start 151 94) (end 151.62 94) (width 0.6) (layer "F.Cu") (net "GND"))
 (segment (start 134.0375 95) (end 135 95) (width 0.6) (layer "F.Cu") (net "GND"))
 (segment (start 121.5 91.5) (end 119 94) (width 0.6) (layer "F.Cu") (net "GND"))
 (segment (start 130.5 62.5) (end 123.5 62.5) (width 0.6) (layer "F.Cu") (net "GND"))
 (segment (start 130.5 65.85) (end 130.5 62.5) (width 0.6) (layer "F.Cu") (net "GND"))
 (segment (start 148.5 96.5) (end 151 94) (width 0.6) (layer "F.Cu") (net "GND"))
 (segment (start 144 96.5) (end 148.5 96.5) (width 0.6) (layer "F.Cu") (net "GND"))
 (segment (start 119 94) (end 117 94) (width 0.6) (layer "F.Cu") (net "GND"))
 (segment (start 123.5 62.5) (end 121.5 64.5) (width 0.6) (layer "F.Cu") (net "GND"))
 (segment (start 143.9 86) (end 150.46 86) (width 0.6) (layer "F.Cu") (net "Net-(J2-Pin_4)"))
 (segment (start 141.095 83.195) (end 143.9 86) (width 0.6) (layer "F.Cu") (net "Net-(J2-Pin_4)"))
 (segment (start 141.095 73.0875) (end 141.095 83.195) (width 0.6) (layer "F.Cu") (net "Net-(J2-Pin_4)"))
 (segment (start 150.46 86) (end 152.5 88.04) (width 0.6) (layer "F.Cu") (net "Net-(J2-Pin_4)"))
 (segment (start 142.365 81.865) (end 142.365 73.0875) (width 0.6) (layer "F.Cu") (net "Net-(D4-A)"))
 (segment (start 145 84.5) (end 142.365 81.865) (width 0.6) (layer "F.Cu") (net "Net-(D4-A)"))
 (segment (start 151.5 84.5) (end 145 84.5) (width 0.6) (layer "F.Cu") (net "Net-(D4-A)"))
 (segment (start 152.5 85.5) (end 151.5 84.5) (width 0.6) (layer "F.Cu") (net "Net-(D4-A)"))
 (segment (start 148.04 82.96) (end 148 83) (width 0.6) (layer "F.Cu") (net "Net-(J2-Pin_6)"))
 (segment (start 148 83) (end 143.635 78.635) (width 0.6) (layer "F.Cu") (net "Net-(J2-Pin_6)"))
 (segment (start 143.635 78.635) (end 143.635 73.0875) (width 0.6) (layer "F.Cu") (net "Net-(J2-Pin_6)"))
 (segment (start 152.5 82.96) (end 148.04 82.96) (width 0.6) (layer "F.Cu") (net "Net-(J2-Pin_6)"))
 (segment (start 131.9625 86.4625) (end 131.9625 95) (width 0.6) (layer "F.Cu") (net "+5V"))
 (segment (start 129 83.5) (end 131.9625 86.4625) (width 0.6) (layer "F.Cu") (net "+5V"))
 (segment (start 129 82.5) (end 129 83.5) (width 0.6) (layer "F.Cu") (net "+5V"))
 (segment (start 144.905 72.179316) (end 144.905 73.0875) (width 0.6) (layer "F.Cu") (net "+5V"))
 (segment (start 129 82.5) (end 140.025 71.475) (width 0.6) (layer "F.Cu") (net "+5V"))
 (segment (start 127 100.25) (end 127 96.5) (width 0.6) (layer "F.Cu") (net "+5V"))
 (segment (start 128.25 101.5) (end 135 101.5) (width 0.6) (layer "F.Cu") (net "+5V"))
 (segment (start 131.3625 95.6) (end 131.9625 95) (width 0.6) (layer "F.Cu") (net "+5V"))
 (segment (start 127.9 95.6) (end 131.3625 95.6) (width 0.6) (layer "F.Cu") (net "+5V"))
 (segment (start 128.25 101.5) (end 127 100.25) (width 0.6) (layer "F.Cu") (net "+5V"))
 (segment (start 140.025 71.475) (end 144.200684 71.475) (width 0.6) (layer "F.Cu") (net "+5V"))
 (segment (start 127 96.5) (end 127.9 95.6) (width 0.6) (layer "F.Cu") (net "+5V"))
 (segment (start 144.200684 71.475) (end 144.905 72.179316) (width 0.6) (layer "F.Cu") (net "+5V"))
 (segment (start 146.16 102) (end 152.5 95.66) (width 0.6) (layer "F.Cu") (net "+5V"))
 (segment (start 135 101.5) (end 135.5 102) (width 0.6) (layer "F.Cu") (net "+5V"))
 (segment (start 135.5 102) (end 146.16 102) (width 0.6) (layer "F.Cu") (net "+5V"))
 (segment (start 144 98.5) (end 136.2 98.5) (width 0.6) (layer "F.Cu") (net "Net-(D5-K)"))
 (segment (start 136.2 98.5) (end 135.5 99.2) (width 0.6) (layer "F.Cu") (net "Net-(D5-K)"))
 (segment (start 140.3 92) (end 145 87.3) (width 0.6) (layer "F.Cu") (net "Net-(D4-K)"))
 (segment (start 139.5 92) (end 140.3 92) (width 0.6) (layer "F.Cu") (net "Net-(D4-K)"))
 (segment (start 121.5 101.5) (end 124.75 101.5) (width 0.6) (layer "F.Cu") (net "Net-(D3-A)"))
 (segment (start 117 101) (end 121 101) (width 0.6) (layer "F.Cu") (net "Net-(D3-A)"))
 (segment (start 121 101) (end 121.5 101.5) (width 0.6) (layer "F.Cu") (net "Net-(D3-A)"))
 (segment (start 125.5 96.444366) (end 125.5 98.5) (width 0.6) (layer "F.Cu") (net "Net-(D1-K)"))
 (segment (start 128.5 94.35) (end 127.594366 94.35) (width 0.6) (layer "F.Cu") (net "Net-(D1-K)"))
 (segment (start 127.594366 94.35) (end 125.5 96.444366) (width 0.6) (layer "F.Cu") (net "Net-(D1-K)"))
 (segment (start 127 82.5) (end 127 92.85) (width 0.6) (layer "F.Cu") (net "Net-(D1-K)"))
 (segment (start 127 77) (end 127 82) (width 0.6) (layer "F.Cu") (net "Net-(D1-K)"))
 (segment (start 127 92.85) (end 128.5 94.35) (width 0.6) (layer "F.Cu") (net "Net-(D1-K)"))
 (segment (start 125.5 98.5) (end 117.5 98.5) (width 0.6) (layer "F.Cu") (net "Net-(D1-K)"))
 (segment (start 122.6 94.5) (end 120.6 96.5) (width 0.6) (layer "F.Cu") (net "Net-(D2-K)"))
 (segment (start 126 68.5) (end 122.6 71.9) (width 0.6) (layer "F.Cu") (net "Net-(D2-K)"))
 (segment (start 126 68.5) (end 129.85 68.5) (width 0.6) (layer "F.Cu") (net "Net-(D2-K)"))
 (segment (start 122.6 71.9) (end 122.6 94.5) (width 0.6) (layer "F.Cu") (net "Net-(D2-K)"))
 (segment (start 120.6 96.5) (end 117.5 96.5) (width 0.6) (layer "F.Cu") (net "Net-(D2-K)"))
 (segment (start 129.85 68.5) (end 130.5 69.15) (width 0.6) (layer "F.Cu") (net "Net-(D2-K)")))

